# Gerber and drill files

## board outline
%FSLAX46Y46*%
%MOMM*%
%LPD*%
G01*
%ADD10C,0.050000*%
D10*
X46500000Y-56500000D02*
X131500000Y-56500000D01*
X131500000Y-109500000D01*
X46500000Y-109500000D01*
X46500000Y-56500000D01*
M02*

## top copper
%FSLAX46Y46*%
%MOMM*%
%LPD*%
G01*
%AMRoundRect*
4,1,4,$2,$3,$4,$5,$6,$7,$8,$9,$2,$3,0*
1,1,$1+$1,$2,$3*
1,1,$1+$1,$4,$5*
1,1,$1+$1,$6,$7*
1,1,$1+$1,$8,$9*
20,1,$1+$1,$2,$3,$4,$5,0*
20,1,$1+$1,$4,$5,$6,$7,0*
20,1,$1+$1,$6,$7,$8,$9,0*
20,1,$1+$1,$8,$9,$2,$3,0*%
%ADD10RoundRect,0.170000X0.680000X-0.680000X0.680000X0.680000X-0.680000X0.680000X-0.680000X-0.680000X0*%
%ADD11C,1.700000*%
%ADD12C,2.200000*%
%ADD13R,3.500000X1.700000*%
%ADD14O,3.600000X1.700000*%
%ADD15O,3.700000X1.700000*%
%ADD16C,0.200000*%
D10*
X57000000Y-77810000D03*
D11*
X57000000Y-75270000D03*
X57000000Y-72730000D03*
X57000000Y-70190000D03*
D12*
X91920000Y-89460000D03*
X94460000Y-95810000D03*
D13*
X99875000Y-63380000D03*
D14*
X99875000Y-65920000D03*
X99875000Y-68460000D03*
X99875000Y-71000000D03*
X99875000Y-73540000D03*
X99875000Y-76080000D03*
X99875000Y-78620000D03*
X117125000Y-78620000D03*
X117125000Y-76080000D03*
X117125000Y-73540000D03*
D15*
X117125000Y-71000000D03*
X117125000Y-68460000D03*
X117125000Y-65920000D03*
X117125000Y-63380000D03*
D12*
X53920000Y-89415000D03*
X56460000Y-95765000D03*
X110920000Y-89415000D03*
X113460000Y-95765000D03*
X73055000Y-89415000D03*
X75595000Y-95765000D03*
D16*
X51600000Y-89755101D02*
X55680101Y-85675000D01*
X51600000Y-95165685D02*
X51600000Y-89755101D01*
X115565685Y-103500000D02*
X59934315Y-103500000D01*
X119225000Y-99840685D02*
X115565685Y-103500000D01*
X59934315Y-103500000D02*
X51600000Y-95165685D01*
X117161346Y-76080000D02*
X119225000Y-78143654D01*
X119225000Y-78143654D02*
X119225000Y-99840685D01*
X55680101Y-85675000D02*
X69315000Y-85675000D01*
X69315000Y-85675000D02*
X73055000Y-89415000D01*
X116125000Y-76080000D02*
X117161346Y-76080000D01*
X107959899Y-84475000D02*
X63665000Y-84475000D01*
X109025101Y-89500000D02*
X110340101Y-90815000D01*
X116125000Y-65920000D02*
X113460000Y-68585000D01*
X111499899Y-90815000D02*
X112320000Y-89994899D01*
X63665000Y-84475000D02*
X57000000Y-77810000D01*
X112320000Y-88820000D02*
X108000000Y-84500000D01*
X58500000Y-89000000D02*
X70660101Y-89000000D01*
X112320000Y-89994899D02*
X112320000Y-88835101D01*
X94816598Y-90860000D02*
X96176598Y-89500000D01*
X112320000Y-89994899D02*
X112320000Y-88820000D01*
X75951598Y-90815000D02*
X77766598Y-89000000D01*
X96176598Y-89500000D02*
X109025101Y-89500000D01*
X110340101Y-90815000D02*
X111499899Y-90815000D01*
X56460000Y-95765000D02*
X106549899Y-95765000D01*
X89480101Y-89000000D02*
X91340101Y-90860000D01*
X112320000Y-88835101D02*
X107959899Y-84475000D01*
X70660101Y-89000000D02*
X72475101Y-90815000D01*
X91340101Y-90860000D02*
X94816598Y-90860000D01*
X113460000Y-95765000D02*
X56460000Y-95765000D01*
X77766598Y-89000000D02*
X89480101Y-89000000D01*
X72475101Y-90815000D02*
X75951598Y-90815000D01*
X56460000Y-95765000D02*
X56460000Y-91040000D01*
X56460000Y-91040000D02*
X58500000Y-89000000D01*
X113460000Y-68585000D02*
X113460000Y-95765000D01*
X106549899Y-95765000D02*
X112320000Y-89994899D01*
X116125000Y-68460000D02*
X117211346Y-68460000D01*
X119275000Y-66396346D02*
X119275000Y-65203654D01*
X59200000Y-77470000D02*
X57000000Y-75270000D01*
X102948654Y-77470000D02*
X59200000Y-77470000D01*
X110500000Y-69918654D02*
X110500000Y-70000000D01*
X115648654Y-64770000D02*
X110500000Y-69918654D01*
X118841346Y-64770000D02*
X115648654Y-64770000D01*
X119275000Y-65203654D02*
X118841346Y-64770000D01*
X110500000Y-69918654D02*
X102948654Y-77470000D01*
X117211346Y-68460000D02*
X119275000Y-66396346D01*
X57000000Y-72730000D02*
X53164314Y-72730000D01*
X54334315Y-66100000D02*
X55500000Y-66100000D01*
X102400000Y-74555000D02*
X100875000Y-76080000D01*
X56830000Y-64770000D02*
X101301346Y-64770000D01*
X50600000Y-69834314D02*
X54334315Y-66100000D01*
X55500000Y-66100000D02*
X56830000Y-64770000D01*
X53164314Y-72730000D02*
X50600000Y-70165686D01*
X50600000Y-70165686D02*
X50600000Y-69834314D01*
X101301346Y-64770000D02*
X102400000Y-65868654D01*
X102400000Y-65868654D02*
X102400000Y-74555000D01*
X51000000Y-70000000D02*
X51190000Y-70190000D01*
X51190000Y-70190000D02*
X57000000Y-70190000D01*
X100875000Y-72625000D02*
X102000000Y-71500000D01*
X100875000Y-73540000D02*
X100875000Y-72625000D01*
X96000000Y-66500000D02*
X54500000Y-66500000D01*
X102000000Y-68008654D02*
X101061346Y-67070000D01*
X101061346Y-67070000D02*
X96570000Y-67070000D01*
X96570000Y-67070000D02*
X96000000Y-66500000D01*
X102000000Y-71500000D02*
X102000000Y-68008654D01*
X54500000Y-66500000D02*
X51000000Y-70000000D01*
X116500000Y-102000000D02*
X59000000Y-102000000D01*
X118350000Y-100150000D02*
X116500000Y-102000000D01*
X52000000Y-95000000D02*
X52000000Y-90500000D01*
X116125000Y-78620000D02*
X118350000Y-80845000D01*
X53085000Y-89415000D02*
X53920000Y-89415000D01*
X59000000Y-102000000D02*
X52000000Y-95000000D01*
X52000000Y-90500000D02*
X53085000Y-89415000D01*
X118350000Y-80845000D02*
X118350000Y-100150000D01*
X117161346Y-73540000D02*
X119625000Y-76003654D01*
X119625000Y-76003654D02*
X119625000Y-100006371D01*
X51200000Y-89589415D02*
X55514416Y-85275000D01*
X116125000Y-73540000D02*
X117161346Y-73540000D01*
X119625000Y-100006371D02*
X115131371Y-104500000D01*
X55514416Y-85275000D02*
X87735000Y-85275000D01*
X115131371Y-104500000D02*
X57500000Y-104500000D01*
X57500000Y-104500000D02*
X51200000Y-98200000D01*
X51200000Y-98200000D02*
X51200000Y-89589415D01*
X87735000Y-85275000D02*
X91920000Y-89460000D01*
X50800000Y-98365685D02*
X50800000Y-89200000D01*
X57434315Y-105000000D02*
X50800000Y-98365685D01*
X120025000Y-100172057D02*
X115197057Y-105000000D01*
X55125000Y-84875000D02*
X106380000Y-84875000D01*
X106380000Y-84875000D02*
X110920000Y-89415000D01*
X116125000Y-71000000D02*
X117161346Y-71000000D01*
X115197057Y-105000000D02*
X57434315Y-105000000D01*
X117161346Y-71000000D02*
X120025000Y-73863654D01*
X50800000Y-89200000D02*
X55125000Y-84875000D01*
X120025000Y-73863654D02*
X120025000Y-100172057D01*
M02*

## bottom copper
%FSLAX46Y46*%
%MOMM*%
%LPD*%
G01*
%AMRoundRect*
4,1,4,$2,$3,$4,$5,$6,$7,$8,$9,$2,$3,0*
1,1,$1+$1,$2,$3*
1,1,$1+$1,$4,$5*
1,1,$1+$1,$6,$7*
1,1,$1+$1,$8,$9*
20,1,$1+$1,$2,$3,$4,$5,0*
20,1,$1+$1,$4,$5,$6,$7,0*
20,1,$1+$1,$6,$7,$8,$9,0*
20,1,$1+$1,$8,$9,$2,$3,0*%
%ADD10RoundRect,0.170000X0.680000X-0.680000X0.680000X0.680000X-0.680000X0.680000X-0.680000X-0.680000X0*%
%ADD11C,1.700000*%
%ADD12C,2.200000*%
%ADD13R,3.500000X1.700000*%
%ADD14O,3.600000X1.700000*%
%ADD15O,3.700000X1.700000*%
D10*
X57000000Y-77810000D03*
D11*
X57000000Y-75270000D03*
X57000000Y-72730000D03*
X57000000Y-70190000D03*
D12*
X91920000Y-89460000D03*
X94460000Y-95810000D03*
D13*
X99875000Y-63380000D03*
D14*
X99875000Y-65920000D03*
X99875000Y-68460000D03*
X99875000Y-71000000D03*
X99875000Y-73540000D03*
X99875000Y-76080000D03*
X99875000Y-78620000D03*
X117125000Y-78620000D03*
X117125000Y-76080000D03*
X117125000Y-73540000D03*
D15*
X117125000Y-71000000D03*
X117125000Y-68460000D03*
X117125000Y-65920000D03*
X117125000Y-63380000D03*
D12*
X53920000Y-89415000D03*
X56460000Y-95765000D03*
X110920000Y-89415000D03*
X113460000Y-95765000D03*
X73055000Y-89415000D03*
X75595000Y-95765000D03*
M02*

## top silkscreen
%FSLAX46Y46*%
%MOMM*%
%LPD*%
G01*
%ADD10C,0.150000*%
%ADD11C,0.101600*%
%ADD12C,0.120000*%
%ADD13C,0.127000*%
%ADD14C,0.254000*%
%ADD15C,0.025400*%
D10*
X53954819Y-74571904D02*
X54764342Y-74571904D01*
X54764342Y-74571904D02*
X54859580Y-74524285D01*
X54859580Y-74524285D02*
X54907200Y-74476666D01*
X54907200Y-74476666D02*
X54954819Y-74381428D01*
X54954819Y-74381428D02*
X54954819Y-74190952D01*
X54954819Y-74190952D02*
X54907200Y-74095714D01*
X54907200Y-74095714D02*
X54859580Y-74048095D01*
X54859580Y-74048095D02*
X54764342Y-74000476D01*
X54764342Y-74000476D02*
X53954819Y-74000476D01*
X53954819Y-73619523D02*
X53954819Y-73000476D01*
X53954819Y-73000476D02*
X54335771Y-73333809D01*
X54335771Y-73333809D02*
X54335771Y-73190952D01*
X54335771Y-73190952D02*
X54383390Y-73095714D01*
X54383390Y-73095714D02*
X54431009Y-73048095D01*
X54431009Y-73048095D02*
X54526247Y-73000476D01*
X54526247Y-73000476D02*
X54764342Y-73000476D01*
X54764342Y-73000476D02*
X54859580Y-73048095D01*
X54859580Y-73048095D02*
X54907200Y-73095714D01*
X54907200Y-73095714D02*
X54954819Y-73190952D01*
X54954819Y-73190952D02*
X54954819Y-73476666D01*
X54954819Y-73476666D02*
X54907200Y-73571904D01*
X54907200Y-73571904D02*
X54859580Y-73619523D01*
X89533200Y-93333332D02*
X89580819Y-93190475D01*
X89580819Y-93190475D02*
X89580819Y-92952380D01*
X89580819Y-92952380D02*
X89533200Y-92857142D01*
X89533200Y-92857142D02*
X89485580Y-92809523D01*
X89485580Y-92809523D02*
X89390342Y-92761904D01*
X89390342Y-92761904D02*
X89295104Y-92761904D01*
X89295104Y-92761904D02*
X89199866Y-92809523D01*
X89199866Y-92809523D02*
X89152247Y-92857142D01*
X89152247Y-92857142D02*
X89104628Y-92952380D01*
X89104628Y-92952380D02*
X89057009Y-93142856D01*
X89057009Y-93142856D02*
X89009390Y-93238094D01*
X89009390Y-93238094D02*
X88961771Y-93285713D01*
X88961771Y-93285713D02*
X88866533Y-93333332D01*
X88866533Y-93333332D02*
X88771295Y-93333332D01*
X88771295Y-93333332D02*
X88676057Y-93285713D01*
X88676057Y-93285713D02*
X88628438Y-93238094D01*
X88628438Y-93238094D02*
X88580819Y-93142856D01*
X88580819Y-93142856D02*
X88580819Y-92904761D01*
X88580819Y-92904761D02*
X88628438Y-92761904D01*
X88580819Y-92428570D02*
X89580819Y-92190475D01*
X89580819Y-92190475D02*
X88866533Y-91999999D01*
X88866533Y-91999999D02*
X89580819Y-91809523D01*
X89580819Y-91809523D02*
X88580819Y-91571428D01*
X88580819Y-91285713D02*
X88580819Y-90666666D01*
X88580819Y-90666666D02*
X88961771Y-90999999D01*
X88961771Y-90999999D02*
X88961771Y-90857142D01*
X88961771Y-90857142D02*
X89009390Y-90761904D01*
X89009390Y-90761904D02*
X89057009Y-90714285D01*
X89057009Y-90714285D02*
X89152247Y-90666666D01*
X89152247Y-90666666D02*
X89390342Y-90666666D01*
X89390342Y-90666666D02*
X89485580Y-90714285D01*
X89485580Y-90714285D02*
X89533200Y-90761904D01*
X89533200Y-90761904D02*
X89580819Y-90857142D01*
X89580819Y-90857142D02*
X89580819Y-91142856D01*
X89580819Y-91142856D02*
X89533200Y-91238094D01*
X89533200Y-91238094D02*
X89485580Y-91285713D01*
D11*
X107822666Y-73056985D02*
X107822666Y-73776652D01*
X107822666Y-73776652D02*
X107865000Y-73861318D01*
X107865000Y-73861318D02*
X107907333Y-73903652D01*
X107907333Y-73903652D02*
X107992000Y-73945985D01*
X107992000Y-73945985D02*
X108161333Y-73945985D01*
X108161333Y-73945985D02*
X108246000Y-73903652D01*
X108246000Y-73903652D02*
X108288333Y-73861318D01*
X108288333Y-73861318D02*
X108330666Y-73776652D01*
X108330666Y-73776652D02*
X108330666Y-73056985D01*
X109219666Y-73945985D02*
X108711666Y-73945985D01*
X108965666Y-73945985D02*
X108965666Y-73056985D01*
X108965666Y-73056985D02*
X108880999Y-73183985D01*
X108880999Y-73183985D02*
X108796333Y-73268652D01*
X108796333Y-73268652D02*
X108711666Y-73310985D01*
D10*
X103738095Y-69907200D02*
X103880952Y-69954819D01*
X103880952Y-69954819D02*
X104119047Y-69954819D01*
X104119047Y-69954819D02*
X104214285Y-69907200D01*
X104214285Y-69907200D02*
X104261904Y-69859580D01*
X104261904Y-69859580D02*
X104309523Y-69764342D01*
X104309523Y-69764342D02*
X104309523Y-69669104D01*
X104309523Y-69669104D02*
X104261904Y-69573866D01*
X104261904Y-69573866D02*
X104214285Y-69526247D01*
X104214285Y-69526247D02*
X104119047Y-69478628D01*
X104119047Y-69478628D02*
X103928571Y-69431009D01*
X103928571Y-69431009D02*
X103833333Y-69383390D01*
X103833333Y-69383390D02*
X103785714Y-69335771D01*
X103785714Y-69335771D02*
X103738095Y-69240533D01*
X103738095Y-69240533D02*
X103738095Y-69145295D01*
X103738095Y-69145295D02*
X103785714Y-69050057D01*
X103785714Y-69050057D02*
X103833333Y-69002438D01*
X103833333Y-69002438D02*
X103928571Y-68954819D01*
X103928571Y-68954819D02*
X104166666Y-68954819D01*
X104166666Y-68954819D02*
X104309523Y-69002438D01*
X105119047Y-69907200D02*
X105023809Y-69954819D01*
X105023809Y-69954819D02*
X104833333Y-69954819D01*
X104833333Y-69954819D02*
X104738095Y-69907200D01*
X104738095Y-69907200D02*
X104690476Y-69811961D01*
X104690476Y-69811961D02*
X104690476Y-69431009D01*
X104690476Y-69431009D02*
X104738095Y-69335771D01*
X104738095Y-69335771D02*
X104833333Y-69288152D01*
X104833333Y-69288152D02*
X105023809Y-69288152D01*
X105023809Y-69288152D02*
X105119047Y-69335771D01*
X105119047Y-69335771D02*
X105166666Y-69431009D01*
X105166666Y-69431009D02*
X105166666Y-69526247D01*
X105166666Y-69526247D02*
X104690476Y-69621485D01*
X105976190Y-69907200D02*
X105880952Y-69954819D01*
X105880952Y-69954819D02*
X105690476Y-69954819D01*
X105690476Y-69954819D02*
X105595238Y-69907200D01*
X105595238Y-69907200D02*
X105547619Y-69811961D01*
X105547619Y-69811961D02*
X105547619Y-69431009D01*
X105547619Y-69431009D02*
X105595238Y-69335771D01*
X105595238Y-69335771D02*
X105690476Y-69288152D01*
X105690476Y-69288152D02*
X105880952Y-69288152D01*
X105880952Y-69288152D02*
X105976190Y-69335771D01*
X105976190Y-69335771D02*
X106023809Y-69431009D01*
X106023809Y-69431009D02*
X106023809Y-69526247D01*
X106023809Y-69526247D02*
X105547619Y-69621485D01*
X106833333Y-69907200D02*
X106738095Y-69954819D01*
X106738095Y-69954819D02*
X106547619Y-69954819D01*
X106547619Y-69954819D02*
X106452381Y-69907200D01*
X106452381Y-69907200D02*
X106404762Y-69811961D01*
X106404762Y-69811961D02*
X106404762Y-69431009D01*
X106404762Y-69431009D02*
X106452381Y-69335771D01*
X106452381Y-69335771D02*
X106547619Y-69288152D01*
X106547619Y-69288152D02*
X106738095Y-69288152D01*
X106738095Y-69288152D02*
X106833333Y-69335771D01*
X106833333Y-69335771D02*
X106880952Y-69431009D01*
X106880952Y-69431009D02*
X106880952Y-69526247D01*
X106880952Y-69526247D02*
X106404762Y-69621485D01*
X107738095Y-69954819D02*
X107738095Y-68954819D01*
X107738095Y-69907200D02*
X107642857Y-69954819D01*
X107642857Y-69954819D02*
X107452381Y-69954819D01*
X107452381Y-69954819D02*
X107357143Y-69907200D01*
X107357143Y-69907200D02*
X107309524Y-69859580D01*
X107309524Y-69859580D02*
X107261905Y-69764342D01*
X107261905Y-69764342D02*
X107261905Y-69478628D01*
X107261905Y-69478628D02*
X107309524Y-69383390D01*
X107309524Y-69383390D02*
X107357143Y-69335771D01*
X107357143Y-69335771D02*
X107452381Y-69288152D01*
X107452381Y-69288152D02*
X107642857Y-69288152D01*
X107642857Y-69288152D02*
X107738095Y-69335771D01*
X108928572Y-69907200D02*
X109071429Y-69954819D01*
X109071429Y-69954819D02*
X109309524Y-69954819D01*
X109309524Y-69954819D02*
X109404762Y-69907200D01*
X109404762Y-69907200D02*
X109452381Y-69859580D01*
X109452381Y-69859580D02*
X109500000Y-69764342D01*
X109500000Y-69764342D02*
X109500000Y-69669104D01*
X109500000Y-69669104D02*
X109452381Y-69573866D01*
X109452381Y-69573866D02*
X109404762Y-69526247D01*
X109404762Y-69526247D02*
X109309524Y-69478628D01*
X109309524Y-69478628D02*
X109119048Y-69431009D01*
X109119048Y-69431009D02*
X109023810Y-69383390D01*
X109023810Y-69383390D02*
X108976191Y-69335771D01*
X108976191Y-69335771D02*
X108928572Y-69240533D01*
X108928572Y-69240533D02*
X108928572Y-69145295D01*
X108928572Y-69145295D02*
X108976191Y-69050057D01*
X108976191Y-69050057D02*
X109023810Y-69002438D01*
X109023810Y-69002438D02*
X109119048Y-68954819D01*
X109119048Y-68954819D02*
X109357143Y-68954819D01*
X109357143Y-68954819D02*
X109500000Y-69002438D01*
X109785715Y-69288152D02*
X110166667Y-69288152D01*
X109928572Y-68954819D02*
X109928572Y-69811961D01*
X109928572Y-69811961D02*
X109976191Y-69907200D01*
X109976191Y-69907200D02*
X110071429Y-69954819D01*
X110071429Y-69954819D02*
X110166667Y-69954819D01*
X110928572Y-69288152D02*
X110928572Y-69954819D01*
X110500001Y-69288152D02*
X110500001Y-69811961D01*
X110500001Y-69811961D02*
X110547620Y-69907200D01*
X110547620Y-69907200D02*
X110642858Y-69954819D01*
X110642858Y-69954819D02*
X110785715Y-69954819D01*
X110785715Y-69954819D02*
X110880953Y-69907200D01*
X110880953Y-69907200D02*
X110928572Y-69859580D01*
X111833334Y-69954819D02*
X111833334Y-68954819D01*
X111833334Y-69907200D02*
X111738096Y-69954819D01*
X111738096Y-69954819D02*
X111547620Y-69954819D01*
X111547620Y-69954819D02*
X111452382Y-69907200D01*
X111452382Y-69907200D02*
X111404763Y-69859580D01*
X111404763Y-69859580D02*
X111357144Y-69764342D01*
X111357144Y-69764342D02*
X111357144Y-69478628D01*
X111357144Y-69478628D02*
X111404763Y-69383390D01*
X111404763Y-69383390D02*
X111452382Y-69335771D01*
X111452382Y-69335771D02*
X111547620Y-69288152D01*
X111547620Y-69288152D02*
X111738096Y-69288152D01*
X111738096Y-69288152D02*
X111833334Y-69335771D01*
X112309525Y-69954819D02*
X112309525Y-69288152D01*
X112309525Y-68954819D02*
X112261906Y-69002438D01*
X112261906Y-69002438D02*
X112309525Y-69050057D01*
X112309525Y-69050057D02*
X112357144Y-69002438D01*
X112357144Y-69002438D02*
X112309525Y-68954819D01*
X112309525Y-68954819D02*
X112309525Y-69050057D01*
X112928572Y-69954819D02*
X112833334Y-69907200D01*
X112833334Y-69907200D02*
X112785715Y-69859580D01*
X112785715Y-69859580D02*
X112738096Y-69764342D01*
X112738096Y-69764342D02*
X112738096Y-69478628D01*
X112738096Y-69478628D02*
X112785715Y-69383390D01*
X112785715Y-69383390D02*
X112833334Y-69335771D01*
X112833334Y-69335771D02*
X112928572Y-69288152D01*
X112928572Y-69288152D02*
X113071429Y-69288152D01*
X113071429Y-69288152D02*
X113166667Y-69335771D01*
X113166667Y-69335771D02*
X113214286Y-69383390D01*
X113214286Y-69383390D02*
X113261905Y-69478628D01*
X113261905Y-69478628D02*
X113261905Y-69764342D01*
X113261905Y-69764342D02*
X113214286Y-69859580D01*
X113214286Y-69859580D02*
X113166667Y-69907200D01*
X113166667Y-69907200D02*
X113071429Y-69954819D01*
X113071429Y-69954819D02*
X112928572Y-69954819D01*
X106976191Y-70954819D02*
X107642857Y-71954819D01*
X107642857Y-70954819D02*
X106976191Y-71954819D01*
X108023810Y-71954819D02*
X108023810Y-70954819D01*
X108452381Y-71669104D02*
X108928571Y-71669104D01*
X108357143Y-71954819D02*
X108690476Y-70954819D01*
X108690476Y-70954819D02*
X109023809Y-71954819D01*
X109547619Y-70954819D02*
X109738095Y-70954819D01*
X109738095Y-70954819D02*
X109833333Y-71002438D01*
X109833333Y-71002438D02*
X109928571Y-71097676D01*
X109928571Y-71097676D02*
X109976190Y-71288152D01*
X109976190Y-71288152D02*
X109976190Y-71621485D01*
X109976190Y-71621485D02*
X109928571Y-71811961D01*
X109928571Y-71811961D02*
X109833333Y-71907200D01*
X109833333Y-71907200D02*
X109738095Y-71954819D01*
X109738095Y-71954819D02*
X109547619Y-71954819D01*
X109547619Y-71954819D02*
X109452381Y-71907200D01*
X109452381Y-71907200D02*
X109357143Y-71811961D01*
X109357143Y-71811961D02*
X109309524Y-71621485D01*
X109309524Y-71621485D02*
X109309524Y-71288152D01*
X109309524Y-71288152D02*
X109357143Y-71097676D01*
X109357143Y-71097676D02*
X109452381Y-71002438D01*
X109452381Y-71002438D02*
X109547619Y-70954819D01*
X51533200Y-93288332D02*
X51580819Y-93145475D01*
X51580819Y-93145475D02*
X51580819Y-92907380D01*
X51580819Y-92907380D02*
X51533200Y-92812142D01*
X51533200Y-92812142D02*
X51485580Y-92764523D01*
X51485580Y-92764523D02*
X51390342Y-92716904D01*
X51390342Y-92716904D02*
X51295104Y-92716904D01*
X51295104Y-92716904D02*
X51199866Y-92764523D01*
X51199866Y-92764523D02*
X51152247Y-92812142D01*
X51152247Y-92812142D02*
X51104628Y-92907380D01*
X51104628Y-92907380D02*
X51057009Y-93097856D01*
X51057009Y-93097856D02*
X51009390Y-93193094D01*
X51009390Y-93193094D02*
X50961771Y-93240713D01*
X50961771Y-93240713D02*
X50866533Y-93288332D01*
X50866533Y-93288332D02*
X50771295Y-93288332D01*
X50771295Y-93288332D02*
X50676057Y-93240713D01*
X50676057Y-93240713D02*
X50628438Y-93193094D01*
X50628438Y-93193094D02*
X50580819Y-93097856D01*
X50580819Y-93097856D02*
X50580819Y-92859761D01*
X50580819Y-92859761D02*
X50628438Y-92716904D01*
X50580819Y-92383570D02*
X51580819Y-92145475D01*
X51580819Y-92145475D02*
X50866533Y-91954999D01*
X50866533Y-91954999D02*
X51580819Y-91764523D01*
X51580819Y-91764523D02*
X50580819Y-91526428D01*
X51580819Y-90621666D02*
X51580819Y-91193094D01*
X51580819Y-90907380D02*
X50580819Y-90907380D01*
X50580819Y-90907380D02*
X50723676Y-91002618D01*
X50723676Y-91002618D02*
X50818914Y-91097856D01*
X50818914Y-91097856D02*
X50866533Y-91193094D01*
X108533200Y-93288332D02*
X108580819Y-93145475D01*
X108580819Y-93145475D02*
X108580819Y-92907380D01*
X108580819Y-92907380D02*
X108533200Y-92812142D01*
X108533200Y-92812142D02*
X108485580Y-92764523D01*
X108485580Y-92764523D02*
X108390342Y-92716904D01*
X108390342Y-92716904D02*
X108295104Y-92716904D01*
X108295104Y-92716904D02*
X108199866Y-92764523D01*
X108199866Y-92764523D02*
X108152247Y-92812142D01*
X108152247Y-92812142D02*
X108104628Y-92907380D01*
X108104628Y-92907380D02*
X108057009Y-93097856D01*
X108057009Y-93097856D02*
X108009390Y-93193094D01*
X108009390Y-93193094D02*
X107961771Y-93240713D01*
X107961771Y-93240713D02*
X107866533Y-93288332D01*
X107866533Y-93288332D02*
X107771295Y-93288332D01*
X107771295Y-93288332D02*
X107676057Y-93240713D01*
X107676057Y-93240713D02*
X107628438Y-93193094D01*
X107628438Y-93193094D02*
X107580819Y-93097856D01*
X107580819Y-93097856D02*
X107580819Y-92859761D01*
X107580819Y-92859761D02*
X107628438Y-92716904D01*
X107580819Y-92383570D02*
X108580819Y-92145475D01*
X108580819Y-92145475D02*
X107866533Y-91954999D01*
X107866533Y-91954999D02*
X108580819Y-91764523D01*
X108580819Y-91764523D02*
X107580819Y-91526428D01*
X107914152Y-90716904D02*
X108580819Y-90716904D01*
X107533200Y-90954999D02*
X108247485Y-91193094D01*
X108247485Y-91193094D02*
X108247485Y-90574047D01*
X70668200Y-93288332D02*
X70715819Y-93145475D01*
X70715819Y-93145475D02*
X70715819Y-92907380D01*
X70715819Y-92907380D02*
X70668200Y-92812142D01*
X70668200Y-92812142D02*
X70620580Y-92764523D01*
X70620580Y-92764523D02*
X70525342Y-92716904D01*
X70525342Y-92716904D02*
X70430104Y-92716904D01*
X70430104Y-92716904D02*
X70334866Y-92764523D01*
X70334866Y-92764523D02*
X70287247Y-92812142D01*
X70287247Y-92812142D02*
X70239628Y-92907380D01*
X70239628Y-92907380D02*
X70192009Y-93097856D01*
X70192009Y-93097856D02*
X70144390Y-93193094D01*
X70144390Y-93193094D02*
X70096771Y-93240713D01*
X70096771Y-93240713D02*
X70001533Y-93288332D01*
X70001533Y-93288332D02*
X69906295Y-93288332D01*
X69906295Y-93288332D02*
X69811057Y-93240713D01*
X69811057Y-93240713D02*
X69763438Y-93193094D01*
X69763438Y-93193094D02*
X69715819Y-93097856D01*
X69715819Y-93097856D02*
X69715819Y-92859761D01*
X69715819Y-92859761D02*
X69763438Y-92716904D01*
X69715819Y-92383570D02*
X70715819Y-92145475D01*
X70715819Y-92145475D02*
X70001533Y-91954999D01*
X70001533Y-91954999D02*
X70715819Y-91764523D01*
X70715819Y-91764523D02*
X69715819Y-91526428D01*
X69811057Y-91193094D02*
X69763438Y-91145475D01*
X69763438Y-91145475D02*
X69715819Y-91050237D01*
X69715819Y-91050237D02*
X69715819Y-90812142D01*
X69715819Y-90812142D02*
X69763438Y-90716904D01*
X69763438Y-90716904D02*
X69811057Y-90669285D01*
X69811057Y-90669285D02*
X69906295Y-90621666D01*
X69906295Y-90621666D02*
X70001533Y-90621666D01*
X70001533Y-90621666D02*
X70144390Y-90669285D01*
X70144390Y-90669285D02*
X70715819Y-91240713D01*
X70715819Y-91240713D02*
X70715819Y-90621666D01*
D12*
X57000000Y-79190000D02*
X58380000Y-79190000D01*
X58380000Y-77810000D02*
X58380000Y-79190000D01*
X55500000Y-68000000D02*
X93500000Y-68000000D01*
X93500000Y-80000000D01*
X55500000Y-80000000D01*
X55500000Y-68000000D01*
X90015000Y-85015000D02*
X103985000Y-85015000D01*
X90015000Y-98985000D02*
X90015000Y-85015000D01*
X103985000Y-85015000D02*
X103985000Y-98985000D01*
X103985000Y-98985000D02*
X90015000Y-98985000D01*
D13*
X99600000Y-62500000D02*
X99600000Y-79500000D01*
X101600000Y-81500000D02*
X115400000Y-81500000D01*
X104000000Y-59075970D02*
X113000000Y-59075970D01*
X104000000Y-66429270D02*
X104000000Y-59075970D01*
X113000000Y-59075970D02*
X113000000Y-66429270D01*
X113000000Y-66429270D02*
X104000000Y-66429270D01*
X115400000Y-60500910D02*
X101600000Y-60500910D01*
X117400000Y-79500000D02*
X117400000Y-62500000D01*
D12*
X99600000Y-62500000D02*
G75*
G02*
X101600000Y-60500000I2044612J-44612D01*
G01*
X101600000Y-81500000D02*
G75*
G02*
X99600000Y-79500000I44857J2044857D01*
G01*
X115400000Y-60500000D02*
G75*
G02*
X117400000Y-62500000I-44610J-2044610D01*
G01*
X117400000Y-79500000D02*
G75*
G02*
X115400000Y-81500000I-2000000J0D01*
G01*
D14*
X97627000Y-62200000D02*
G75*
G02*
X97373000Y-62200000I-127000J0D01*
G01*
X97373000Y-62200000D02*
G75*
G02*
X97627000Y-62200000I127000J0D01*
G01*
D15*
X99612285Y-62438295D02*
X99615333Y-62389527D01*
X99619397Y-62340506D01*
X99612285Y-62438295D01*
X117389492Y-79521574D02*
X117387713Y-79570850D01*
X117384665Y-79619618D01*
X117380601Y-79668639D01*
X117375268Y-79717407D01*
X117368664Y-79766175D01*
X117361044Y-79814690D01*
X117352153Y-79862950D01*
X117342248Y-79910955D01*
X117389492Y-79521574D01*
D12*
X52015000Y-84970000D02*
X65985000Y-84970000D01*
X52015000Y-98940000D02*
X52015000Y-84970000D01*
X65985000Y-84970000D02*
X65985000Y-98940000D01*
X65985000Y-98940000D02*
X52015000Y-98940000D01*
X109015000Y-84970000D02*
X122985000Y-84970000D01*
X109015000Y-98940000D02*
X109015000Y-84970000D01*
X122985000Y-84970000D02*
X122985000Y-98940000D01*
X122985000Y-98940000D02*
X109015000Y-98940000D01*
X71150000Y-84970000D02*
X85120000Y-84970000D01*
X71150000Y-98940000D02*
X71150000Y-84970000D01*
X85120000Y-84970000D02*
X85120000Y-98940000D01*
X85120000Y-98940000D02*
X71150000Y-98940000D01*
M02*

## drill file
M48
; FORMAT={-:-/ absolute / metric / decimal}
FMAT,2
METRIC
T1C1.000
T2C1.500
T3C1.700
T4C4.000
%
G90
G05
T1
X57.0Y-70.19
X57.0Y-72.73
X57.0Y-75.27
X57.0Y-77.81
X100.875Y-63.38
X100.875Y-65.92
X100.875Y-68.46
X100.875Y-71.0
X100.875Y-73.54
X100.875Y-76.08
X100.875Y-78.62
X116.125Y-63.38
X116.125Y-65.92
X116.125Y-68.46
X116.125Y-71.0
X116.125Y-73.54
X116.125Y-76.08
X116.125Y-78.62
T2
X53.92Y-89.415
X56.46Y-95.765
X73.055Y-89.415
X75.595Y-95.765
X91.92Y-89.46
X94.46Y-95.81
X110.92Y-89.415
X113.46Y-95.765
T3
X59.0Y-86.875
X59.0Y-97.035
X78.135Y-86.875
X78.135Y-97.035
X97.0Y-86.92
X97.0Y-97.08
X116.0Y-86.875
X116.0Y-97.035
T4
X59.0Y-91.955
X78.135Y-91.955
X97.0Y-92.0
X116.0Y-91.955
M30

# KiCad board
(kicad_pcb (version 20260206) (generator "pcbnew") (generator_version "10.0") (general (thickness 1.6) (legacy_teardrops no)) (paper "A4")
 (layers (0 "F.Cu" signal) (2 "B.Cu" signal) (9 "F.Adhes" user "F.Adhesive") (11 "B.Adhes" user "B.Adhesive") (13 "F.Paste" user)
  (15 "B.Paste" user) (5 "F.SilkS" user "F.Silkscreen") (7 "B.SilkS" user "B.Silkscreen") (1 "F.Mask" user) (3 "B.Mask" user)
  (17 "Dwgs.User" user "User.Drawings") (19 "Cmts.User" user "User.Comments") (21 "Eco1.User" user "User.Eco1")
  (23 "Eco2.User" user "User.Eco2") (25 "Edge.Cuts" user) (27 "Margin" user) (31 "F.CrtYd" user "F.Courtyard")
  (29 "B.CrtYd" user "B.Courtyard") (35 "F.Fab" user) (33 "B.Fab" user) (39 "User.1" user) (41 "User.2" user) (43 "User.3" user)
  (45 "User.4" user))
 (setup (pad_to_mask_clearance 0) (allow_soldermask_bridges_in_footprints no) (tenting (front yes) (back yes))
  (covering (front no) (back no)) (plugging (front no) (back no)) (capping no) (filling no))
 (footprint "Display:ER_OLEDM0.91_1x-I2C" (layer "F.Cu") (at 57 77.81 90)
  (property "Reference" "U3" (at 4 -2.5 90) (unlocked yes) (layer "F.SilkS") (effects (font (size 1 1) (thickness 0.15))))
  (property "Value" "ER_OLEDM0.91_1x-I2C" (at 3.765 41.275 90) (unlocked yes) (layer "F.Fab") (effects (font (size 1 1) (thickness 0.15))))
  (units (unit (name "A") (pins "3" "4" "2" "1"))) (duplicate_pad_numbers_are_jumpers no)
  (fp_line (start -1.38 0) (end -1.38 1.38) (stroke (width 0.12) (type solid)) (layer "F.SilkS"))
  (fp_line (start 0 1.38) (end -1.38 1.38) (stroke (width 0.12) (type solid)) (layer "F.SilkS"))
  (fp_rect (start -2.19 -1.5) (end 9.81 36.5) (stroke (width 0.12) (type solid)) (fill no) (layer "F.SilkS"))
  (pad "1" thru_hole roundrect (at 0 0 90) (size 1.7 1.7) (drill 1) (layers "*.Cu" "*.Mask") (remove_unused_layers no)
   (roundrect_rratio 0.1) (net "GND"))
  (pad "2" thru_hole circle (at 2.54 0 90) (size 1.7 1.7) (drill 1) (layers "*.Cu" "*.Mask") (remove_unused_layers no) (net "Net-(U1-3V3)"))
  (pad "3" thru_hole circle (at 5.08 0 90) (size 1.7 1.7) (drill 1) (layers "*.Cu" "*.Mask") (remove_unused_layers no)
   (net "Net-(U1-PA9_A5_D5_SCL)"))
  (pad "4" thru_hole circle (at 7.62 0 90) (size 1.7 1.7) (drill 1) (layers "*.Cu" "*.Mask") (remove_unused_layers no)
   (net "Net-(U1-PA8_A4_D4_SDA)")))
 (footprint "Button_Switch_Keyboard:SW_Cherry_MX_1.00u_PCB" (layer "F.Cu") (at 91.92 89.46 90)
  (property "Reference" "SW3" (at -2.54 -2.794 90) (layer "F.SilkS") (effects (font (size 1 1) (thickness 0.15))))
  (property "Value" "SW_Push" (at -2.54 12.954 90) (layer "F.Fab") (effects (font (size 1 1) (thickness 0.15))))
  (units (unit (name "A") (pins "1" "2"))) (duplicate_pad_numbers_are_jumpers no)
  (fp_line (start 4.445 -1.905) (end 4.445 12.065) (stroke (width 0.12) (type solid)) (layer "F.SilkS"))
  (fp_line (start -9.525 -1.905) (end 4.445 -1.905) (stroke (width 0.12) (type solid)) (layer "F.SilkS"))
  (fp_line (start 4.445 12.065) (end -9.525 12.065) (stroke (width 0.12) (type solid)) (layer "F.SilkS"))
  (fp_line (start -9.525 12.065) (end -9.525 -1.905) (stroke (width 0.12) (type solid)) (layer "F.SilkS"))
  (pad "" np_thru_hole circle (at -7.62 5.08 90) (size 1.7 1.7) (drill 1.7) (layers "*.Cu" "*.Mask"))
  (pad "" np_thru_hole circle (at -2.54 5.08 90) (size 4 4) (drill 4) (layers "*.Cu" "*.Mask"))
  (pad "" np_thru_hole circle (at 2.54 5.08 90) (size 1.7 1.7) (drill 1.7) (layers "*.Cu" "*.Mask"))
  (pad "1" thru_hole circle (at 0 0 90) (size 2.2 2.2) (drill 1.5) (layers "*.Cu" "*.Mask") (remove_unused_layers no)
   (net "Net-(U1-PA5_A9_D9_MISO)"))
  (pad "2" thru_hole circle (at -6.35 2.54 90) (size 2.2 2.2) (drill 1.5) (layers "*.Cu" "*.Mask") (remove_unused_layers no) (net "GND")))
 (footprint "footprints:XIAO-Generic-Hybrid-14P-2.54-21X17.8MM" (layer "F.Cu") (at 108.5 71)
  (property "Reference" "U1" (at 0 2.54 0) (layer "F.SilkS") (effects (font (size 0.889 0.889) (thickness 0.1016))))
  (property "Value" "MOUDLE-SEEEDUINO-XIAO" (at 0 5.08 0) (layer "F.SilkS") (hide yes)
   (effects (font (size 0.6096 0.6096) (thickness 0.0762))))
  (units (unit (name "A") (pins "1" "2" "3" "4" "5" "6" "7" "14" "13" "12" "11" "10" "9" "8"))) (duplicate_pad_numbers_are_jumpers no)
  (fp_line (start -8.9 -8.5) (end -8.9 8.5) (stroke (width 0.127) (type solid)) (layer "F.SilkS"))
  (fp_line (start -6.9 10.5) (end 6.9 10.5) (stroke (width 0.127) (type solid)) (layer "F.SilkS"))
  (fp_line (start -4.5 -11.92403) (end 4.5 -11.92403) (stroke (width 0.127) (type solid)) (layer "F.SilkS"))
  (fp_line (start -4.5 -4.57073) (end -4.5 -11.92403) (stroke (width 0.127) (type solid)) (layer "F.SilkS"))
  (fp_line (start 4.5 -11.92403) (end 4.5 -4.57073) (stroke (width 0.127) (type solid)) (layer "F.SilkS"))
  (fp_line (start 4.5 -4.57073) (end -4.5 -4.57073) (stroke (width 0.127) (type solid)) (layer "F.SilkS"))
  (fp_line (start 6.9 -10.49909) (end -6.9 -10.49909) (stroke (width 0.127) (type solid)) (layer "F.SilkS"))
  (fp_line (start 8.9 8.5) (end 8.9 -8.5) (stroke (width 0.127) (type solid)) (layer "F.SilkS"))
  (fp_arc (start -8.9 -8.5) (mid -8.301491 -9.901491) (end -6.9 -10.5) (stroke (width 0.12) (type solid)) (layer "F.SilkS"))
  (fp_arc (start -6.9 10.5) (mid -8.301423 9.901423) (end -8.9 8.5) (stroke (width 0.12) (type solid)) (layer "F.SilkS"))
  (fp_arc (start 6.9 -10.5) (mid 8.301491 -9.901491) (end 8.9 -8.5) (stroke (width 0.12) (type solid)) (layer "F.SilkS"))
  (fp_arc (start 8.9 8.5) (mid 8.314214 9.914214) (end 6.9 10.5) (stroke (width 0.12) (type solid)) (layer "F.SilkS"))
  (fp_circle (center -11 -8.8) (end -11 -9.054) (stroke (width 0) (type solid)) (fill yes) (layer "F.SilkS"))
  (fp_poly
   (pts (xy -8.887715 -8.561705) (xy -8.884667 -8.610473) (xy -8.880603 -8.659494)) (stroke (width 0.0254) (type solid)) (fill no)
   (layer "F.SilkS"))
  (fp_poly
   (pts (xy 8.889492 8.521574) (xy 8.887713 8.57085) (xy 8.884665 8.619618) (xy 8.880601 8.668639) (xy 8.875268 8.717407)
    (xy 8.868664 8.766175) (xy 8.861044 8.81469) (xy 8.852153 8.86295) (xy 8.842248 8.910955))
   (stroke (width 0.0254) (type solid)) (fill no) (layer "F.SilkS"))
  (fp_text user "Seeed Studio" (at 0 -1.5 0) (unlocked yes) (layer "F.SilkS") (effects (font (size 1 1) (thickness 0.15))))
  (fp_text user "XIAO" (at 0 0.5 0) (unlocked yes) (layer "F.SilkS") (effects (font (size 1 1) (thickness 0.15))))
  (pad "1" thru_hole rect (at -7.625 -7.62) (size 3.5 1.7) (drill 1 (offset -1 0)) (layers "*.Cu" "*.Mask") (remove_unused_layers no)
   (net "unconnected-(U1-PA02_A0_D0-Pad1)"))
  (pad "2" thru_hole oval (at -7.625 -5.08) (size 3.6 1.7) (drill 1 (offset -1 0)) (layers "*.Cu" "*.Mask") (remove_unused_layers no)
   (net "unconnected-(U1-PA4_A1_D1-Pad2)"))
  (pad "3" thru_hole oval (at -7.625 -2.54) (size 3.6 1.7) (drill 1 (offset -1 0)) (layers "*.Cu" "*.Mask") (remove_unused_layers no)
   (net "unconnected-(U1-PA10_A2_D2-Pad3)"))
  (pad "4" thru_hole oval (at -7.625 0) (size 3.6 1.7) (drill 1 (offset -1 0)) (layers "*.Cu" "*.Mask") (remove_unused_layers no)
   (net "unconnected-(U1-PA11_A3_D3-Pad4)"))
  (pad "5" thru_hole oval (at -7.625 2.54) (size 3.6 1.7) (drill 1 (offset -1 0)) (layers "*.Cu" "*.Mask") (remove_unused_layers no)
   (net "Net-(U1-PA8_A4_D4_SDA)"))
  (pad "6" thru_hole oval (at -7.625 5.08 180) (size 3.6 1.7) (drill 1 (offset 1 0)) (layers "*.Cu" "*.Mask") (remove_unused_layers no)
   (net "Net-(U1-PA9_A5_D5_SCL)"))
  (pad "7" thru_hole oval (at -7.625 7.62) (size 3.6 1.7) (drill 1 (offset -1 0)) (layers "*.Cu" "*.Mask") (remove_unused_layers no)
   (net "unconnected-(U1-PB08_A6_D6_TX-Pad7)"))
  (pad "8" thru_hole oval (at 7.625 7.62) (size 3.6 1.7) (drill 1 (offset 1 0)) (layers "*.Cu" "*.Mask") (remove_unused_layers no)
   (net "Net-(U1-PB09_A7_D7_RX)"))
  (pad "9" thru_hole oval (at 7.625 5.08) (size 3.6 1.7) (drill 1 (offset 1 0)) (layers "*.Cu" "*.Mask") (remove_unused_layers no)
   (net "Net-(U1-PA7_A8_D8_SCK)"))
  (pad "10" thru_hole oval (at 7.625 2.54) (size 3.6 1.7) (drill 1 (offset 1 0)) (layers "*.Cu" "*.Mask") (remove_unused_layers no)
   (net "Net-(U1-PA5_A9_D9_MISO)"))
  (pad "11" thru_hole oval (at 7.625 0) (size 3.7 1.7) (drill 1 (offset 1 0)) (layers "*.Cu" "*.Mask") (remove_unused_layers no)
   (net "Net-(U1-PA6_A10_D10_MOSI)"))
  (pad "12" thru_hole oval (at 7.625 -2.54) (size 3.7 1.7) (drill 1 (offset 1 0)) (layers "*.Cu" "*.Mask") (remove_unused_layers no)
   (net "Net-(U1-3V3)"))
  (pad "13" thru_hole oval (at 7.625 -5.08) (size 3.7 1.7) (drill 1 (offset 1 0)) (layers "*.Cu" "*.Mask") (remove_unused_layers no)
   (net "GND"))
  (pad "14" thru_hole oval (at 7.625 -7.62) (size 3.7 1.7) (drill 1 (offset 1 0)) (layers "*.Cu" "*.Mask") (remove_unused_layers no)
   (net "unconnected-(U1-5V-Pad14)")))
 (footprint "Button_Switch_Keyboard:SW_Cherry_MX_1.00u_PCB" (layer "F.Cu") (at 53.92 89.415 90)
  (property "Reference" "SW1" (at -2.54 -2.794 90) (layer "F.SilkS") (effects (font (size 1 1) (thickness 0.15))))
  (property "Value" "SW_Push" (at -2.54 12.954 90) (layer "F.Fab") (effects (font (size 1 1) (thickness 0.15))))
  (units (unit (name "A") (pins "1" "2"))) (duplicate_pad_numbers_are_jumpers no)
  (fp_line (start 4.445 -1.905) (end 4.445 12.065) (stroke (width 0.12) (type solid)) (layer "F.SilkS"))
  (fp_line (start -9.525 -1.905) (end 4.445 -1.905) (stroke (width 0.12) (type solid)) (layer "F.SilkS"))
  (fp_line (start 4.445 12.065) (end -9.525 12.065) (stroke (width 0.12) (type solid)) (layer "F.SilkS"))
  (fp_line (start -9.525 12.065) (end -9.525 -1.905) (stroke (width 0.12) (type solid)) (layer "F.SilkS"))
  (pad "" np_thru_hole circle (at -7.62 5.08 90) (size 1.7 1.7) (drill 1.7) (layers "*.Cu" "*.Mask"))
  (pad "" np_thru_hole circle (at -2.54 5.08 90) (size 4 4) (drill 4) (layers "*.Cu" "*.Mask"))
  (pad "" np_thru_hole circle (at 2.54 5.08 90) (size 1.7 1.7) (drill 1.7) (layers "*.Cu" "*.Mask"))
  (pad "1" thru_hole circle (at 0 0 90) (size 2.2 2.2) (drill 1.5) (layers "*.Cu" "*.Mask") (remove_unused_layers no)
   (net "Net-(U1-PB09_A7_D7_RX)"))
  (pad "2" thru_hole circle (at -6.35 2.54 90) (size 2.2 2.2) (drill 1.5) (layers "*.Cu" "*.Mask") (remove_unused_layers no) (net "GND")))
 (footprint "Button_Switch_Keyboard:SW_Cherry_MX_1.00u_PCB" (layer "F.Cu") (at 110.92 89.415 90)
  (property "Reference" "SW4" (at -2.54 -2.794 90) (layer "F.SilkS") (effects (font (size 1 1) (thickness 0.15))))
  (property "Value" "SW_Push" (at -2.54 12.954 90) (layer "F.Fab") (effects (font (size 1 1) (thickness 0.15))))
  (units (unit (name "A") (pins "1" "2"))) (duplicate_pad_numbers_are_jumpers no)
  (fp_line (start 4.445 -1.905) (end 4.445 12.065) (stroke (width 0.12) (type solid)) (layer "F.SilkS"))
  (fp_line (start -9.525 -1.905) (end 4.445 -1.905) (stroke (width 0.12) (type solid)) (layer "F.SilkS"))
  (fp_line (start 4.445 12.065) (end -9.525 12.065) (stroke (width 0.12) (type solid)) (layer "F.SilkS"))
  (fp_line (start -9.525 12.065) (end -9.525 -1.905) (stroke (width 0.12) (type solid)) (layer "F.SilkS"))
  (pad "" np_thru_hole circle (at -7.62 5.08 90) (size 1.7 1.7) (drill 1.7) (layers "*.Cu" "*.Mask"))
  (pad "" np_thru_hole circle (at -2.54 5.08 90) (size 4 4) (drill 4) (layers "*.Cu" "*.Mask"))
  (pad "" np_thru_hole circle (at 2.54 5.08 90) (size 1.7 1.7) (drill 1.7) (layers "*.Cu" "*.Mask"))
  (pad "1" thru_hole circle (at 0 0 90) (size 2.2 2.2) (drill 1.5) (layers "*.Cu" "*.Mask") (remove_unused_layers no)
   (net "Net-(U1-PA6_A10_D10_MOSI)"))
  (pad "2" thru_hole circle (at -6.35 2.54 90) (size 2.2 2.2) (drill 1.5) (layers "*.Cu" "*.Mask") (remove_unused_layers no) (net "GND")))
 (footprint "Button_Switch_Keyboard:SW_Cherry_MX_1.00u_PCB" (layer "F.Cu") (at 73.055 89.415 90)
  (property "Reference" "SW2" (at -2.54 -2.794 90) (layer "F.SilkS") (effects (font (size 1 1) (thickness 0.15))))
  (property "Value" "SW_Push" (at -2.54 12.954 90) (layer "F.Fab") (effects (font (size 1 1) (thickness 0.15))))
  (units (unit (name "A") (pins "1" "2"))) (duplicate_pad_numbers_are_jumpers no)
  (fp_line (start 4.445 -1.905) (end 4.445 12.065) (stroke (width 0.12) (type solid)) (layer "F.SilkS"))
  (fp_line (start -9.525 -1.905) (end 4.445 -1.905) (stroke (width 0.12) (type solid)) (layer "F.SilkS"))
  (fp_line (start 4.445 12.065) (end -9.525 12.065) (stroke (width 0.12) (type solid)) (layer "F.SilkS"))
  (fp_line (start -9.525 12.065) (end -9.525 -1.905) (stroke (width 0.12) (type solid)) (layer "F.SilkS"))
  (pad "" np_thru_hole circle (at -7.62 5.08 90) (size 1.7 1.7) (drill 1.7) (layers "*.Cu" "*.Mask"))
  (pad "" np_thru_hole circle (at -2.54 5.08 90) (size 4 4) (drill 4) (layers "*.Cu" "*.Mask"))
  (pad "" np_thru_hole circle (at 2.54 5.08 90) (size 1.7 1.7) (drill 1.7) (layers "*.Cu" "*.Mask"))
  (pad "1" thru_hole circle (at 0 0 90) (size 2.2 2.2) (drill 1.5) (layers "*.Cu" "*.Mask") (remove_unused_layers no)
   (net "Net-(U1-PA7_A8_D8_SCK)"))
  (pad "2" thru_hole circle (at -6.35 2.54 90) (size 2.2 2.2) (drill 1.5) (layers "*.Cu" "*.Mask") (remove_unused_layers no) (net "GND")))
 (gr_rect (start 46.5 56.5) (end 131.5 109.5) (stroke (width 0.05) (type default)) (fill no) (layer "Edge.Cuts"))
 (segment (start 51.6 89.755101) (end 55.680101 85.675) (width 0.2) (layer "F.Cu") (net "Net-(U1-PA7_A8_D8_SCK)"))
 (segment (start 51.6 95.165685) (end 51.6 89.755101) (width 0.2) (layer "F.Cu") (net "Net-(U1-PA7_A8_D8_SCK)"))
 (segment (start 115.565685 103.5) (end 59.934315 103.5) (width 0.2) (layer "F.Cu") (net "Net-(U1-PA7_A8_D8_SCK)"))
 (segment (start 119.225 99.840685) (end 115.565685 103.5) (width 0.2) (layer "F.Cu") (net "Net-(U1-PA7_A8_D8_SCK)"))
 (segment (start 59.934315 103.5) (end 51.6 95.165685) (width 0.2) (layer "F.Cu") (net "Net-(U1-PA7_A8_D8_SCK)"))
 (segment (start 117.161346 76.08) (end 119.225 78.143654) (width 0.2) (layer "F.Cu") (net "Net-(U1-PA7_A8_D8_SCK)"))
 (segment (start 119.225 78.143654) (end 119.225 99.840685) (width 0.2) (layer "F.Cu") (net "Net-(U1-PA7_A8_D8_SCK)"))
 (segment (start 55.680101 85.675) (end 69.315 85.675) (width 0.2) (layer "F.Cu") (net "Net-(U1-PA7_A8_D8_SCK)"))
 (segment (start 69.315 85.675) (end 73.055 89.415) (width 0.2) (layer "F.Cu") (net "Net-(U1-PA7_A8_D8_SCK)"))
 (segment (start 116.125 76.08) (end 117.161346 76.08) (width 0.2) (layer "F.Cu") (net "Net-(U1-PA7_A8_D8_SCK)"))
 (segment (start 107.959899 84.475) (end 63.665 84.475) (width 0.2) (layer "F.Cu") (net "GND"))
 (segment (start 109.025101 89.5) (end 110.340101 90.815) (width 0.2) (layer "F.Cu") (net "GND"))
 (segment (start 116.125 65.92) (end 113.46 68.585) (width 0.2) (layer "F.Cu") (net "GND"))
 (segment (start 111.499899 90.815) (end 112.32 89.994899) (width 0.2) (layer "F.Cu") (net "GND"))
 (segment (start 63.665 84.475) (end 57 77.81) (width 0.2) (layer "F.Cu") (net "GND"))
 (segment (start 112.32 88.82) (end 108 84.5) (width 0.2) (layer "F.Cu") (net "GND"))
 (segment (start 58.5 89) (end 70.660101 89) (width 0.2) (layer "F.Cu") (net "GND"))
 (segment (start 112.32 89.994899) (end 112.32 88.835101) (width 0.2) (layer "F.Cu") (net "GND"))
 (segment (start 94.816598 90.86) (end 96.176598 89.5) (width 0.2) (layer "F.Cu") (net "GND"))
 (segment (start 112.32 89.994899) (end 112.32 88.82) (width 0.2) (layer "F.Cu") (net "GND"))
 (segment (start 75.951598 90.815) (end 77.766598 89) (width 0.2) (layer "F.Cu") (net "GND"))
 (segment (start 96.176598 89.5) (end 109.025101 89.5) (width 0.2) (layer "F.Cu") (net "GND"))
 (segment (start 110.340101 90.815) (end 111.499899 90.815) (width 0.2) (layer "F.Cu") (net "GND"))
 (segment (start 56.46 95.765) (end 106.549899 95.765) (width 0.2) (layer "F.Cu") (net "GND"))
 (segment (start 89.480101 89) (end 91.340101 90.86) (width 0.2) (layer "F.Cu") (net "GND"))
 (segment (start 112.32 88.835101) (end 107.959899 84.475) (width 0.2) (layer "F.Cu") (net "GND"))
 (segment (start 70.660101 89) (end 72.475101 90.815) (width 0.2) (layer "F.Cu") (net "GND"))
 (segment (start 91.340101 90.86) (end 94.816598 90.86) (width 0.2) (layer "F.Cu") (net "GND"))
 (segment (start 113.46 95.765) (end 56.46 95.765) (width 0.2) (layer "F.Cu") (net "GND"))
 (segment (start 77.766598 89) (end 89.480101 89) (width 0.2) (layer "F.Cu") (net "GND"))
 (segment (start 72.475101 90.815) (end 75.951598 90.815) (width 0.2) (layer "F.Cu") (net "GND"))
 (segment (start 56.46 95.765) (end 56.46 91.04) (width 0.2) (layer "F.Cu") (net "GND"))
 (segment (start 56.46 91.04) (end 58.5 89) (width 0.2) (layer "F.Cu") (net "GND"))
 (segment (start 113.46 68.585) (end 113.46 95.765) (width 0.2) (layer "F.Cu") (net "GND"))
 (segment (start 106.549899 95.765) (end 112.32 89.994899) (width 0.2) (layer "F.Cu") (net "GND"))
 (segment (start 116.125 68.46) (end 117.211346 68.46) (width 0.2) (layer "F.Cu") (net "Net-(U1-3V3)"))
 (segment (start 119.275 66.396346) (end 119.275 65.203654) (width 0.2) (layer "F.Cu") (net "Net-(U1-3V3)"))
 (segment (start 59.2 77.47) (end 57 75.27) (width 0.2) (layer "F.Cu") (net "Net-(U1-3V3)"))
 (segment (start 102.948654 77.47) (end 59.2 77.47) (width 0.2) (layer "F.Cu") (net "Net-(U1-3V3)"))
 (segment (start 110.5 69.918654) (end 110.5 70) (width 0.2) (layer "F.Cu") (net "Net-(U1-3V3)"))
 (segment (start 115.648654 64.77) (end 110.5 69.918654) (width 0.2) (layer "F.Cu") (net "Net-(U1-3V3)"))
 (segment (start 118.841346 64.77) (end 115.648654 64.77) (width 0.2) (layer "F.Cu") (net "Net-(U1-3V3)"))
 (segment (start 119.275 65.203654) (end 118.841346 64.77) (width 0.2) (layer "F.Cu") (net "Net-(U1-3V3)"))
 (segment (start 110.5 69.918654) (end 102.948654 77.47) (width 0.2) (layer "F.Cu") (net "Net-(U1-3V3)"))
 (segment (start 117.211346 68.46) (end 119.275 66.396346) (width 0.2) (layer "F.Cu") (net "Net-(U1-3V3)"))
 (segment (start 57 72.73) (end 53.164314 72.73) (width 0.2) (layer "F.Cu") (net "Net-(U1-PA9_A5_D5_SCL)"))
 (segment (start 54.334315 66.1) (end 55.5 66.1) (width 0.2) (layer "F.Cu") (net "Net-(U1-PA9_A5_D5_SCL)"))
 (segment (start 102.4 74.555) (end 100.875 76.08) (width 0.2) (layer "F.Cu") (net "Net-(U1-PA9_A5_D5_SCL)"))
 (segment (start 56.83 64.77) (end 101.301346 64.77) (width 0.2) (layer "F.Cu") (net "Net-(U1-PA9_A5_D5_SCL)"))
 (segment (start 50.6 69.834314) (end 54.334315 66.1) (width 0.2) (layer "F.Cu") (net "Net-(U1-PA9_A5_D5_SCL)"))
 (segment (start 55.5 66.1) (end 56.83 64.77) (width 0.2) (layer "F.Cu") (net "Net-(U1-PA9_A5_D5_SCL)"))
 (segment (start 53.164314 72.73) (end 50.6 70.165686) (width 0.2) (layer "F.Cu") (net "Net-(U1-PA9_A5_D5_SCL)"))
 (segment (start 50.6 70.165686) (end 50.6 69.834314) (width 0.2) (layer "F.Cu") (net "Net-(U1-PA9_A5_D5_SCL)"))
 (segment (start 101.301346 64.77) (end 102.4 65.868654) (width 0.2) (layer "F.Cu") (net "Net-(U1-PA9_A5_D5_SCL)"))
 (segment (start 102.4 65.868654) (end 102.4 74.555) (width 0.2) (layer "F.Cu") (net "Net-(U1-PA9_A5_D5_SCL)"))
 (segment (start 51 70) (end 51.19 70.19) (width 0.2) (layer "F.Cu") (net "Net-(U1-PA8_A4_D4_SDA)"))
 (segment (start 51.19 70.19) (end 57 70.19) (width 0.2) (layer "F.Cu") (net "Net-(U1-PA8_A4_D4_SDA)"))
 (segment (start 100.875 72.625) (end 102 71.5) (width 0.2) (layer "F.Cu") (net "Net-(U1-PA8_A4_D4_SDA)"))
 (segment (start 100.875 73.54) (end 100.875 72.625) (width 0.2) (layer "F.Cu") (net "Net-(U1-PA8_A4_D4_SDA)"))
 (segment (start 96 66.5) (end 54.5 66.5) (width 0.2) (layer "F.Cu") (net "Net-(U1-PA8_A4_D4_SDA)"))
 (segment (start 102 68.008654) (end 101.061346 67.07) (width 0.2) (layer "F.Cu") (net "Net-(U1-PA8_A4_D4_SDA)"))
 (segment (start 101.061346 67.07) (end 96.57 67.07) (width 0.2) (layer "F.Cu") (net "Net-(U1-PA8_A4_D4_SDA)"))
 (segment (start 96.57 67.07) (end 96 66.5) (width 0.2) (layer "F.Cu") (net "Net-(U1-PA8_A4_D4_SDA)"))
 (segment (start 102 71.5) (end 102 68.008654) (width 0.2) (layer "F.Cu") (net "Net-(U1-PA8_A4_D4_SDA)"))
 (segment (start 54.5 66.5) (end 51 70) (width 0.2) (layer "F.Cu") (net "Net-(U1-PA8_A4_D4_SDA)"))
 (segment (start 116.5 102) (end 59 102) (width 0.2) (layer "F.Cu") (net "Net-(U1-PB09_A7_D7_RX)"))
 (segment (start 118.35 100.15) (end 116.5 102) (width 0.2) (layer "F.Cu") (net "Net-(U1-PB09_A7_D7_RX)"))
 (segment (start 52 95) (end 52 90.5) (width 0.2) (layer "F.Cu") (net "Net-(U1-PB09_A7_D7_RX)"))
 (segment (start 116.125 78.62) (end 118.35 80.845) (width 0.2) (layer "F.Cu") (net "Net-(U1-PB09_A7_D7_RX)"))
 (segment (start 53.085 89.415) (end 53.92 89.415) (width 0.2) (layer "F.Cu") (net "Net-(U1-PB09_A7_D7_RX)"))
 (segment (start 59 102) (end 52 95) (width 0.2) (layer "F.Cu") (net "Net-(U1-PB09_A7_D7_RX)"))
 (segment (start 52 90.5) (end 53.085 89.415) (width 0.2) (layer "F.Cu") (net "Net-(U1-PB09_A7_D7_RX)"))
 (segment (start 118.35 80.845) (end 118.35 100.15) (width 0.2) (layer "F.Cu") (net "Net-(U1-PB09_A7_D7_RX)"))
 (segment (start 117.161346 73.54) (end 119.625 76.003654) (width 0.2) (layer "F.Cu") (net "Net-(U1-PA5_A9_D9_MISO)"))
 (segment (start 119.625 76.003654) (end 119.625 100.006371) (width 0.2) (layer "F.Cu") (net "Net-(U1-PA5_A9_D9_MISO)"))
 (segment (start 51.2 89.589415) (end 55.514416 85.275) (width 0.2) (layer "F.Cu") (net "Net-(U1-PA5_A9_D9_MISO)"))
 (segment (start 116.125 73.54) (end 117.161346 73.54) (width 0.2) (layer "F.Cu") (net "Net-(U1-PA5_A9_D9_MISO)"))
 (segment (start 119.625 100.006371) (end 115.131371 104.5) (width 0.2) (layer "F.Cu") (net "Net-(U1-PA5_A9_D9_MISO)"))
 (segment (start 55.514416 85.275) (end 87.735 85.275) (width 0.2) (layer "F.Cu") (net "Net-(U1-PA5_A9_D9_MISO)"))
 (segment (start 115.131371 104.5) (end 57.5 104.5) (width 0.2) (layer "F.Cu") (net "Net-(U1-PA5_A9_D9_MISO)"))
 (segment (start 57.5 104.5) (end 51.2 98.2) (width 0.2) (layer "F.Cu") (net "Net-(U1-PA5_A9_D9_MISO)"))
 (segment (start 51.2 98.2) (end 51.2 89.589415) (width 0.2) (layer "F.Cu") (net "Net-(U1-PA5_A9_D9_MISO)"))
 (segment (start 87.735 85.275) (end 91.92 89.46) (width 0.2) (layer "F.Cu") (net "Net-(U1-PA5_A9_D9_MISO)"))
 (segment (start 50.8 98.365685) (end 50.8 89.2) (width 0.2) (layer "F.Cu") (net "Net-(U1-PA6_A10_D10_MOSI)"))
 (segment (start 57.434315 105) (end 50.8 98.365685) (width 0.2) (layer "F.Cu") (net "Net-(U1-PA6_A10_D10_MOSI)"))
 (segment (start 120.025 100.172057) (end 115.197057 105) (width 0.2) (layer "F.Cu") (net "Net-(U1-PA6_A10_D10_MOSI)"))
 (segment (start 55.125 84.875) (end 106.38 84.875) (width 0.2) (layer "F.Cu") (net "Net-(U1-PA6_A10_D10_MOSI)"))
 (segment (start 106.38 84.875) (end 110.92 89.415) (width 0.2) (layer "F.Cu") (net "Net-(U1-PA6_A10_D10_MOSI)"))
 (segment (start 116.125 71) (end 117.161346 71) (width 0.2) (layer "F.Cu") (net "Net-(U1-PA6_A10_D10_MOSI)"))
 (segment (start 115.197057 105) (end 57.434315 105) (width 0.2) (layer "F.Cu") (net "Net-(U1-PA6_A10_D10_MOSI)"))
 (segment (start 117.161346 71) (end 120.025 73.863654) (width 0.2) (layer "F.Cu") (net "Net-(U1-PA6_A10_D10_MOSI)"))
 (segment (start 50.8 89.2) (end 55.125 84.875) (width 0.2) (layer "F.Cu") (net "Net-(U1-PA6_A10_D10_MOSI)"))
 (segment (start 120.025 73.863654) (end 120.025 100.172057) (width 0.2) (layer "F.Cu") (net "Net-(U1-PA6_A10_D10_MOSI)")))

